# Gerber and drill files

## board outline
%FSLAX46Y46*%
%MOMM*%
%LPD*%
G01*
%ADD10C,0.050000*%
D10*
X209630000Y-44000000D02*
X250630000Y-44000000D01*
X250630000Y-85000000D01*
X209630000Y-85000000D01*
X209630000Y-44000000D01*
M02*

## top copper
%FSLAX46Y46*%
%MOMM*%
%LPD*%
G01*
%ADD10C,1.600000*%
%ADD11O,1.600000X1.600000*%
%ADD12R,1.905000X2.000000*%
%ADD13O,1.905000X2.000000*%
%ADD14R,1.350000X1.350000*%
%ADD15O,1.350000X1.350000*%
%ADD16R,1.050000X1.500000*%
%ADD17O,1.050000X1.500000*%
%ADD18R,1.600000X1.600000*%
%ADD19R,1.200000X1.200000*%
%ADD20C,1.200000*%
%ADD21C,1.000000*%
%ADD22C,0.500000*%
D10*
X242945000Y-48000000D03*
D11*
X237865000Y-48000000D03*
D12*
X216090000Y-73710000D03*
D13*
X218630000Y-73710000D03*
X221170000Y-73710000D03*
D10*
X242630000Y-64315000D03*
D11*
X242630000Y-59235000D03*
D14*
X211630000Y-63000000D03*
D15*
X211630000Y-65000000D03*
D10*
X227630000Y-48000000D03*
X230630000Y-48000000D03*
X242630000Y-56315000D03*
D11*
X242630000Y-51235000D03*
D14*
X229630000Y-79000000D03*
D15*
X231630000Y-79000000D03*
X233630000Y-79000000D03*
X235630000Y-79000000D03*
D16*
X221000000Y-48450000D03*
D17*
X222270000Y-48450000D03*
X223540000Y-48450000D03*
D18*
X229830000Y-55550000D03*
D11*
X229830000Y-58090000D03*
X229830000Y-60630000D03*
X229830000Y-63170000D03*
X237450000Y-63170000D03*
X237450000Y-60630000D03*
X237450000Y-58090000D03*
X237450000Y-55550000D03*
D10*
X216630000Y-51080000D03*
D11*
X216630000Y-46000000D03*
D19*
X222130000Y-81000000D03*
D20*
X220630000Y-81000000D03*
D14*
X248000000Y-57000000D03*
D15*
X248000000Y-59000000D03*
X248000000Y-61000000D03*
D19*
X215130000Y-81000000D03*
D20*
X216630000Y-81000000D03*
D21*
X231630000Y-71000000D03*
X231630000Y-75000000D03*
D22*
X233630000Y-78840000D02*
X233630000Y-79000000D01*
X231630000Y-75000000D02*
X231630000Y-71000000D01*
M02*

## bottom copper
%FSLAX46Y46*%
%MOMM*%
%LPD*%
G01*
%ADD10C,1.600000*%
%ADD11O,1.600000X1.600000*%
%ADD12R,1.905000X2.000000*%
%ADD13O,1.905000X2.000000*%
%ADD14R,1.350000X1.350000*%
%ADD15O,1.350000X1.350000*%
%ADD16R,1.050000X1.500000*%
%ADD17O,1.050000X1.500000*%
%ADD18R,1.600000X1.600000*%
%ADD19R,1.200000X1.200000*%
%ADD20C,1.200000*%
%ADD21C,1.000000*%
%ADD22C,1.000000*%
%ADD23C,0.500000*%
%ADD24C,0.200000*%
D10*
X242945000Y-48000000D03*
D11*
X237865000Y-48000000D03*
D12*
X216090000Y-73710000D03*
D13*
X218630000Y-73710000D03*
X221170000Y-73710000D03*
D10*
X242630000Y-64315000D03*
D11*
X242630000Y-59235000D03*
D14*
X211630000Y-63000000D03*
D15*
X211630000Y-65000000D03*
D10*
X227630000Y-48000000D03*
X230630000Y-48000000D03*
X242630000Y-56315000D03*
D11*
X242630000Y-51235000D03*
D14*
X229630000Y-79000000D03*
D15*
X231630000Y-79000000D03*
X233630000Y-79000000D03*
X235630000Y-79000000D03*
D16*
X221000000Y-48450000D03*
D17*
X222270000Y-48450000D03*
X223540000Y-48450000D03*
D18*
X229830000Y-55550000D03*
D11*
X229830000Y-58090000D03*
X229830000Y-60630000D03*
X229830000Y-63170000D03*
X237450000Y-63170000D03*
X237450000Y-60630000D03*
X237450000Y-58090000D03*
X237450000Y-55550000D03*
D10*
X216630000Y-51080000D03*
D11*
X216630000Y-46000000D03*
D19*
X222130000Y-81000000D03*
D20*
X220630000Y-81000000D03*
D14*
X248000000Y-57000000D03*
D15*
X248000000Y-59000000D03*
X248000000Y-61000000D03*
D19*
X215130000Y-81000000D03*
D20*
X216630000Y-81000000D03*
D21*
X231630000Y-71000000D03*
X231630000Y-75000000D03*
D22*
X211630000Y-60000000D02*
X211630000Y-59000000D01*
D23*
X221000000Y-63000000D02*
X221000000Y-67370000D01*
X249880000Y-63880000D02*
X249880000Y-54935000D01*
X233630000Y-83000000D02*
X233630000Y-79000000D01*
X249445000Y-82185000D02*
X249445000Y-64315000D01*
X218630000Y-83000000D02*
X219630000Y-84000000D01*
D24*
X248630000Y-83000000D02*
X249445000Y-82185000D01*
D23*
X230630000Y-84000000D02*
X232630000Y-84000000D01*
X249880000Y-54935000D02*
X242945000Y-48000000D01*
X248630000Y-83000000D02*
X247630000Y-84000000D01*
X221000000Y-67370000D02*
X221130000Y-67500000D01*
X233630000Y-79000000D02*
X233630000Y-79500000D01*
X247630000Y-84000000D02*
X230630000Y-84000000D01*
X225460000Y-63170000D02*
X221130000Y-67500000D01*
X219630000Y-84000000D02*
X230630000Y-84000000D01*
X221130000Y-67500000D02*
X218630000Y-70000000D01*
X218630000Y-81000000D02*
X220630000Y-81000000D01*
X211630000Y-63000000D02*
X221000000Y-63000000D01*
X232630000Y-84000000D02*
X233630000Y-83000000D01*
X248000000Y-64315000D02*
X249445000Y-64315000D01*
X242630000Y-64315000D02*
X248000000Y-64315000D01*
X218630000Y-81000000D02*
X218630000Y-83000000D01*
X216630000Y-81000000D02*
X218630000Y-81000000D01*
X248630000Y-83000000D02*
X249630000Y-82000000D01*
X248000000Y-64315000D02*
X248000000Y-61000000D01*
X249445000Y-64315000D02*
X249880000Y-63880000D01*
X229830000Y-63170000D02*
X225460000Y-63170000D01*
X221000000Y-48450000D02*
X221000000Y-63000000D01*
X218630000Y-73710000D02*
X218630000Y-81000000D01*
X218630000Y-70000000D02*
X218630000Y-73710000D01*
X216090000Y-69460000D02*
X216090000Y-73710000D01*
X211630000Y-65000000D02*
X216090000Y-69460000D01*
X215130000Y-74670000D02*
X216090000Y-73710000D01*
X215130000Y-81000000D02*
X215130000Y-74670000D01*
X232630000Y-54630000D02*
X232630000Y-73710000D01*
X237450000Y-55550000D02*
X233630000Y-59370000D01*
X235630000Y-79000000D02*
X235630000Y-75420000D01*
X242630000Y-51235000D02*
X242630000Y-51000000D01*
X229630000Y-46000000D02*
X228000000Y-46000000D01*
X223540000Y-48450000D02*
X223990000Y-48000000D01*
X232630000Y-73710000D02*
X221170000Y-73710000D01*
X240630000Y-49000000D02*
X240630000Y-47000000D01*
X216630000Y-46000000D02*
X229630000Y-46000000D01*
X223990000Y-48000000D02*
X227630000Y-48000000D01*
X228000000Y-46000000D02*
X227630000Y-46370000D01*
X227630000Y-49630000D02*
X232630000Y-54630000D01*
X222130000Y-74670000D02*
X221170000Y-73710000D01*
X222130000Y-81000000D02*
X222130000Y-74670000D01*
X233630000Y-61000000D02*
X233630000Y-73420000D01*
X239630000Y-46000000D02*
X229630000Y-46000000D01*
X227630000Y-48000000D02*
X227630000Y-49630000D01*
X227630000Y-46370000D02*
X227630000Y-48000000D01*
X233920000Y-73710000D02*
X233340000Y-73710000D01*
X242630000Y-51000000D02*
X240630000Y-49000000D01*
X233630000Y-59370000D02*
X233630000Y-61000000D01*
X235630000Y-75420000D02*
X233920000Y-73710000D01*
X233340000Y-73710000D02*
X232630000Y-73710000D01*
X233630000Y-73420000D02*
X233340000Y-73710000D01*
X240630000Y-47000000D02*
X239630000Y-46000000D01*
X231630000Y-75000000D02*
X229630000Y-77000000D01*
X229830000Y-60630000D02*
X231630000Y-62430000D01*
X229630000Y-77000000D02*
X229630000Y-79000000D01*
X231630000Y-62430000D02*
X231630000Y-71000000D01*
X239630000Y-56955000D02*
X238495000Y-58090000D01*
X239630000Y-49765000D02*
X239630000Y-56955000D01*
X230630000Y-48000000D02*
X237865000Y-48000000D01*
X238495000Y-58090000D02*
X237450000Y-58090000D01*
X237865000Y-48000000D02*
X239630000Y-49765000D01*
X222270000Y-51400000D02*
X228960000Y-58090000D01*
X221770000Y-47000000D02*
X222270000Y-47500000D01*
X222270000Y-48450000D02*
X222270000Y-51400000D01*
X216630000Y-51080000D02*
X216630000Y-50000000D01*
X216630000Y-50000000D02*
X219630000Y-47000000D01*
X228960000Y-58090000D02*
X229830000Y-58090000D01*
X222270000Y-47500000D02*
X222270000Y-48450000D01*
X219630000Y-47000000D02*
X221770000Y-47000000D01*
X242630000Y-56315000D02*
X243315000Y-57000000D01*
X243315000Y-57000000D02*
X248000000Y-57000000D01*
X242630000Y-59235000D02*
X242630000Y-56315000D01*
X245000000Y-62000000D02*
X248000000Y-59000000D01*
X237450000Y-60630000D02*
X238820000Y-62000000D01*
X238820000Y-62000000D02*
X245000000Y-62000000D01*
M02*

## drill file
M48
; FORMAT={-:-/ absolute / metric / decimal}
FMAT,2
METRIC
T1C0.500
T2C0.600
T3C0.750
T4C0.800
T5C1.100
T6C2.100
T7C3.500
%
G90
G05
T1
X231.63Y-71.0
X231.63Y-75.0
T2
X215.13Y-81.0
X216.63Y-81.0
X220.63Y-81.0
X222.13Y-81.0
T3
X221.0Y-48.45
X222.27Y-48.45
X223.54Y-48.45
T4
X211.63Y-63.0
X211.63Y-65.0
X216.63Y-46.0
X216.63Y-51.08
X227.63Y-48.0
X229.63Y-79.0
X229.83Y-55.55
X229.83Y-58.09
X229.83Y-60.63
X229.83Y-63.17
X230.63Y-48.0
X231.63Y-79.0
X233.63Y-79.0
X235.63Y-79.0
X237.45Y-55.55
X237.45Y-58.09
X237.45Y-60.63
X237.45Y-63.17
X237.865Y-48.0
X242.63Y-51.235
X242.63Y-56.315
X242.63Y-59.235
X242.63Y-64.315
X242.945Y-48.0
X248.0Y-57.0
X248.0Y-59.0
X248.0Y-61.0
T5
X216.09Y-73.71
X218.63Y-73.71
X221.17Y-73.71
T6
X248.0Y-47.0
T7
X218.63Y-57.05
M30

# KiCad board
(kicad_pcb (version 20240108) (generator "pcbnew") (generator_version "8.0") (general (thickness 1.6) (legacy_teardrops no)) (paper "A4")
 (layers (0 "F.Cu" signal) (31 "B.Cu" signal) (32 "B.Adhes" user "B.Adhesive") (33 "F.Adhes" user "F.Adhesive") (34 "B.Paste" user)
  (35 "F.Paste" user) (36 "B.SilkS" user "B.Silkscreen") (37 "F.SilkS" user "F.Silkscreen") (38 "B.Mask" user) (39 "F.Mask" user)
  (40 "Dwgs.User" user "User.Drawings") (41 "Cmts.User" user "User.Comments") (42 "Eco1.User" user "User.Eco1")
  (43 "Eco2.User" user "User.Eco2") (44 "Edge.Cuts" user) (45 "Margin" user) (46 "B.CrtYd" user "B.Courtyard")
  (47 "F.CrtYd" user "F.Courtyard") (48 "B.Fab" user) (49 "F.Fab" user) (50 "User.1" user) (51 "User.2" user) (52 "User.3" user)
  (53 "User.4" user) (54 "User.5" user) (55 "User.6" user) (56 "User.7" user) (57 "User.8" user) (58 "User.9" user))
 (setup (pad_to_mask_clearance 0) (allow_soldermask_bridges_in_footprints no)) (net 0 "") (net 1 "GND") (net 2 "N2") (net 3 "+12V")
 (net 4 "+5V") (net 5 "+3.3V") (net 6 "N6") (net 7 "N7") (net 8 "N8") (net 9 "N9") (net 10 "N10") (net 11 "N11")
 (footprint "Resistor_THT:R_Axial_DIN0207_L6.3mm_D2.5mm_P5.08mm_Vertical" (layer "F.Cu") (at 242.945 48 180)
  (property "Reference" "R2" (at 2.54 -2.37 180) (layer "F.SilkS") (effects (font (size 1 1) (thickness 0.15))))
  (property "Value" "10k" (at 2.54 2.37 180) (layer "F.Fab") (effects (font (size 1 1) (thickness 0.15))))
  (pad "1" thru_hole circle (at 0 0 180) (size 1.6 1.6) (drill 0.8) (layers "*.Cu" "*.Mask") (remove_unused_layers no) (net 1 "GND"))
  (pad "2" thru_hole oval (at 5.08 0 180) (size 1.6 1.6) (drill 0.8) (layers "*.Cu" "*.Mask") (remove_unused_layers no) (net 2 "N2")))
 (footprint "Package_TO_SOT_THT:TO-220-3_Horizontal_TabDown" (layer "F.Cu") (at 216.09 73.71)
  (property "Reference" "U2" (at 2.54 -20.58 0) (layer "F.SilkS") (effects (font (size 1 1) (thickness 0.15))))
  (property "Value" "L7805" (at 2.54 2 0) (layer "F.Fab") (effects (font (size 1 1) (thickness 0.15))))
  (pad "" np_thru_hole oval (at 2.54 -16.66) (size 3.5 3.5) (drill 3.5) (layers "*.Cu" "*.Mask"))
  (pad "1" thru_hole rect (at 0 0) (size 1.905 2) (drill 1.1) (layers "*.Cu" "*.Mask") (remove_unused_layers no) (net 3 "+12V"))
  (pad "2" thru_hole oval (at 2.54 0) (size 1.905 2) (drill 1.1) (layers "*.Cu" "*.Mask") (remove_unused_layers no) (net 1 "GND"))
  (pad "3" thru_hole oval (at 5.08 0) (size 1.905 2) (drill 1.1) (layers "*.Cu" "*.Mask") (remove_unused_layers no) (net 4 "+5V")))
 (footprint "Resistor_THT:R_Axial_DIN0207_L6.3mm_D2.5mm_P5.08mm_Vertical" (layer "F.Cu") (at 242.63 64.315 90)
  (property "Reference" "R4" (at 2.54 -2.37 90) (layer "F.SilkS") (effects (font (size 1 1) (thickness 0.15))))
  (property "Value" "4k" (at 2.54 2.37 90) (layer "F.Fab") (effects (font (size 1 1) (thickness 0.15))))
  (pad "1" thru_hole circle (at 0 0 90) (size 1.6 1.6) (drill 0.8) (layers "*.Cu" "*.Mask") (remove_unused_layers no) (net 1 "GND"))
  (pad "2" thru_hole oval (at 5.08 0 90) (size 1.6 1.6) (drill 0.8) (layers "*.Cu" "*.Mask") (remove_unused_layers no) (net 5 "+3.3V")))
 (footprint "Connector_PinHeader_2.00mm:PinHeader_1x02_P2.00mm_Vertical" (layer "F.Cu") (at 211.63 63)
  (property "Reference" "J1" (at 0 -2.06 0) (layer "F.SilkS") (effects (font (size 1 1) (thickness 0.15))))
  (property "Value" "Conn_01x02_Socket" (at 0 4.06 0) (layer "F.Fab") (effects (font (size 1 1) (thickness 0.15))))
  (pad "1" thru_hole rect (at 0 0) (size 1.35 1.35) (drill 0.8) (layers "*.Cu" "*.Mask") (remove_unused_layers no) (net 1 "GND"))
  (pad "2" thru_hole oval (at 0 2) (size 1.35 1.35) (drill 0.8) (layers "*.Cu" "*.Mask") (remove_unused_layers no) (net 3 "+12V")))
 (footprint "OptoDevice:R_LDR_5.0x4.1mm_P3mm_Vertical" (layer "F.Cu") (at 227.63 48)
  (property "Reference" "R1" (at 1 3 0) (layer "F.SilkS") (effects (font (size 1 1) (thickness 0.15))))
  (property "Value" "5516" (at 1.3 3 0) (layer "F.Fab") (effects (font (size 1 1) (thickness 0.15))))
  (pad "1" thru_hole circle (at 0 0) (size 1.6 1.6) (drill 0.8) (layers "*.Cu" "*.Mask") (remove_unused_layers no) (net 4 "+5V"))
  (pad "2" thru_hole circle (at 3 0) (size 1.6 1.6) (drill 0.8) (layers "*.Cu" "*.Mask") (remove_unused_layers no) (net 2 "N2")))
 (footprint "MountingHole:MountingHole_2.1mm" (layer "F.Cu") (at 248 47)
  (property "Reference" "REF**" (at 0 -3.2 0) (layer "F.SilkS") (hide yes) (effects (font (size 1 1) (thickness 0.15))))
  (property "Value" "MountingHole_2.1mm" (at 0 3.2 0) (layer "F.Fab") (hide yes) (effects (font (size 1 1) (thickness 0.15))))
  (pad "" np_thru_hole circle (at 0 0) (size 2.1 2.1) (drill 2.1) (layers "*.Cu" "*.Mask")))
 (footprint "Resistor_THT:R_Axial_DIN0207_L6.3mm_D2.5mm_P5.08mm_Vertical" (layer "F.Cu") (at 242.63 56.315 90)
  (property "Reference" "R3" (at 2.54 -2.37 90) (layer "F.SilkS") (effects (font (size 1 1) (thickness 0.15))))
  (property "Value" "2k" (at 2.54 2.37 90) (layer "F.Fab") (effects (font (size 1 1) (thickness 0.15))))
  (pad "1" thru_hole circle (at 0 0 90) (size 1.6 1.6) (drill 0.8) (layers "*.Cu" "*.Mask") (remove_unused_layers no) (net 5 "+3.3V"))
  (pad "2" thru_hole oval (at 5.08 0 90) (size 1.6 1.6) (drill 0.8) (layers "*.Cu" "*.Mask") (remove_unused_layers no) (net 4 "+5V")))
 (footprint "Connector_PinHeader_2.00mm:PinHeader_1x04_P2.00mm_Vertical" (layer "F.Cu") (at 229.63 79 90)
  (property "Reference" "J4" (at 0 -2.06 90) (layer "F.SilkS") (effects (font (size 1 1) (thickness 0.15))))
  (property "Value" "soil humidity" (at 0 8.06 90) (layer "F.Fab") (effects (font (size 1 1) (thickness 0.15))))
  (pad "1" thru_hole rect (at 0 0 90) (size 1.35 1.35) (drill 0.8) (layers "*.Cu" "*.Mask") (remove_unused_layers no) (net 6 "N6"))
  (pad "2" thru_hole oval (at 0 2 90) (size 1.35 1.35) (drill 0.8) (layers "*.Cu" "*.Mask") (remove_unused_layers no) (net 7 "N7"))
  (pad "3" thru_hole oval (at 0 4 90) (size 1.35 1.35) (drill 0.8) (layers "*.Cu" "*.Mask") (remove_unused_layers no) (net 1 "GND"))
  (pad "4" thru_hole oval (at 0 6 90) (size 1.35 1.35) (drill 0.8) (layers "*.Cu" "*.Mask") (remove_unused_layers no) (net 4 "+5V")))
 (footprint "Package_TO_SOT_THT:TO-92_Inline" (layer "F.Cu") (at 221 48.45)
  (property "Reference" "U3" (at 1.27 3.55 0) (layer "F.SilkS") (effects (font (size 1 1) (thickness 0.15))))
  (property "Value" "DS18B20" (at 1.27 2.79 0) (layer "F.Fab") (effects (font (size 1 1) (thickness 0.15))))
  (pad "1" thru_hole rect (at 0 0) (size 1.05 1.5) (drill 0.75) (layers "*.Cu" "*.Mask") (remove_unused_layers no) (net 1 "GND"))
  (pad "2" thru_hole oval (at 1.27 0) (size 1.05 1.5) (drill 0.75) (layers "*.Cu" "*.Mask") (remove_unused_layers no) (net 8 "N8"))
  (pad "3" thru_hole oval (at 2.54 0) (size 1.05 1.5) (drill 0.75) (layers "*.Cu" "*.Mask") (remove_unused_layers no) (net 4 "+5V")))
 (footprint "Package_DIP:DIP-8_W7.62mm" (layer "F.Cu") (at 229.83 55.55)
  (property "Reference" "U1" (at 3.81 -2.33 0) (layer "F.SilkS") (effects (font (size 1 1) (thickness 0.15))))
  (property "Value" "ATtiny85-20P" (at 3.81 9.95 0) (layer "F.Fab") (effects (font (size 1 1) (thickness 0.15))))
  (pad "1" thru_hole rect (at 0 0) (size 1.6 1.6) (drill 0.8) (layers "*.Cu" "*.Mask") (remove_unused_layers no) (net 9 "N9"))
  (pad "2" thru_hole oval (at 0 2.54) (size 1.6 1.6) (drill 0.8) (layers "*.Cu" "*.Mask") (remove_unused_layers no) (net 8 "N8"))
  (pad "3" thru_hole oval (at 0 5.08) (size 1.6 1.6) (drill 0.8) (layers "*.Cu" "*.Mask") (remove_unused_layers no) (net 6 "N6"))
  (pad "4" thru_hole oval (at 0 7.62) (size 1.6 1.6) (drill 0.8) (layers "*.Cu" "*.Mask") (remove_unused_layers no) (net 1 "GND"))
  (pad "5" thru_hole oval (at 7.62 7.62) (size 1.6 1.6) (drill 0.8) (layers "*.Cu" "*.Mask") (remove_unused_layers no) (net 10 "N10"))
  (pad "6" thru_hole oval (at 7.62 5.08) (size 1.6 1.6) (drill 0.8) (layers "*.Cu" "*.Mask") (remove_unused_layers no) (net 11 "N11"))
  (pad "7" thru_hole oval (at 7.62 2.54) (size 1.6 1.6) (drill 0.8) (layers "*.Cu" "*.Mask") (remove_unused_layers no) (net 2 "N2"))
  (pad "8" thru_hole oval (at 7.62 0) (size 1.6 1.6) (drill 0.8) (layers "*.Cu" "*.Mask") (remove_unused_layers no) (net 4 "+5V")))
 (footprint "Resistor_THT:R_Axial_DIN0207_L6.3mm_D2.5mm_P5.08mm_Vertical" (layer "F.Cu") (at 216.63 51.08 90)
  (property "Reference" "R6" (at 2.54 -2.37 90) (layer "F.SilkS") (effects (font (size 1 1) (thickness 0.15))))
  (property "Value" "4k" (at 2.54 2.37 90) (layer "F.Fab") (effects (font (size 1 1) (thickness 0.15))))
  (pad "1" thru_hole circle (at 0 0 90) (size 1.6 1.6) (drill 0.8) (layers "*.Cu" "*.Mask") (remove_unused_layers no) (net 8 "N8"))
  (pad "2" thru_hole oval (at 5.08 0 90) (size 1.6 1.6) (drill 0.8) (layers "*.Cu" "*.Mask") (remove_unused_layers no) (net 4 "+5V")))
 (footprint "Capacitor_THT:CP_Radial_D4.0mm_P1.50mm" (layer "F.Cu") (at 222.13 81 180)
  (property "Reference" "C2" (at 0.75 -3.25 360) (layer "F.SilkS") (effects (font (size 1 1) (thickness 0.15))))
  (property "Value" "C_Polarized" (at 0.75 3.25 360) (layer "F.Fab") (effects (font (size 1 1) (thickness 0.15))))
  (pad "1" thru_hole rect (at 0 0 180) (size 1.2 1.2) (drill 0.6) (layers "*.Cu" "*.Mask") (remove_unused_layers no) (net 4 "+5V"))
  (pad "2" thru_hole circle (at 1.5 0 180) (size 1.2 1.2) (drill 0.6) (layers "*.Cu" "*.Mask") (remove_unused_layers no) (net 1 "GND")))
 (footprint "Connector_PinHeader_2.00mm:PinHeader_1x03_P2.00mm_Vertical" (layer "F.Cu") (at 248 57)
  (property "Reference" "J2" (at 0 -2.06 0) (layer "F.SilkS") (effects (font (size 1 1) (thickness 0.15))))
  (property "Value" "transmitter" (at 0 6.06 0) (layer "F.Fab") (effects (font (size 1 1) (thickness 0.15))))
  (pad "1" thru_hole rect (at 0 0) (size 1.35 1.35) (drill 0.8) (layers "*.Cu" "*.Mask") (remove_unused_layers no) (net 5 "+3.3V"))
  (pad "2" thru_hole oval (at 0 2) (size 1.35 1.35) (drill 0.8) (layers "*.Cu" "*.Mask") (remove_unused_layers no) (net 11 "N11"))
  (pad "3" thru_hole oval (at 0 4) (size 1.35 1.35) (drill 0.8) (layers "*.Cu" "*.Mask") (remove_unused_layers no) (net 1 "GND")))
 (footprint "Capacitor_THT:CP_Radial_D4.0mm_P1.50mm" (layer "F.Cu") (at 215.13 81)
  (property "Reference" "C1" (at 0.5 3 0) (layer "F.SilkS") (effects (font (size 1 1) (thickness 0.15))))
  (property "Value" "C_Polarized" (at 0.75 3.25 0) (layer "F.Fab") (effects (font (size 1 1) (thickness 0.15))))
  (pad "1" thru_hole rect (at 0 0) (size 1.2 1.2) (drill 0.6) (layers "*.Cu" "*.Mask") (remove_unused_layers no) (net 3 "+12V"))
  (pad "2" thru_hole circle (at 1.5 0) (size 1.2 1.2) (drill 0.6) (layers "*.Cu" "*.Mask") (remove_unused_layers no) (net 1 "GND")))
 (gr_rect (start 209.63 44) (end 250.63 85) (stroke (width 0.05) (type default)) (fill none) (layer "Edge.Cuts"))
 (segment (start 211.63 60) (end 211.63 59) (width 1) (layer "B.Cu") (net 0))
 (segment (start 233.63 78.84) (end 233.63 79) (width 0.5) (layer "F.Cu") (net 1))
 (segment (start 221 63) (end 221 67.37) (width 0.5) (layer "B.Cu") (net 1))
 (segment (start 249.88 63.88) (end 249.88 54.935) (width 0.5) (layer "B.Cu") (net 1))
 (segment (start 233.63 83) (end 233.63 79) (width 0.5) (layer "B.Cu") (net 1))
 (segment (start 249.445 82.185) (end 249.445 64.315) (width 0.5) (layer "B.Cu") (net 1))
 (segment (start 218.63 83) (end 219.63 84) (width 0.5) (layer "B.Cu") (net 1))
 (segment (start 248.63 83) (end 249.445 82.185) (width 0.2) (layer "B.Cu") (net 1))
 (segment (start 230.63 84) (end 232.63 84) (width 0.5) (layer "B.Cu") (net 1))
 (segment (start 249.88 54.935) (end 242.945 48) (width 0.5) (layer "B.Cu") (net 1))
 (segment (start 248.63 83) (end 247.63 84) (width 0.5) (layer "B.Cu") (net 1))
 (segment (start 221 67.37) (end 221.13 67.5) (width 0.5) (layer "B.Cu") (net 1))
 (segment (start 233.63 79) (end 233.63 79.5) (width 0.5) (layer "B.Cu") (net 1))
 (segment (start 247.63 84) (end 230.63 84) (width 0.5) (layer "B.Cu") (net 1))
 (segment (start 225.46 63.17) (end 221.13 67.5) (width 0.5) (layer "B.Cu") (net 1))
 (segment (start 219.63 84) (end 230.63 84) (width 0.5) (layer "B.Cu") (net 1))
 (segment (start 221.13 67.5) (end 218.63 70) (width 0.5) (layer "B.Cu") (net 1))
 (segment (start 218.63 81) (end 220.63 81) (width 0.5) (layer "B.Cu") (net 1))
 (segment (start 211.63 63) (end 221 63) (width 0.5) (layer "B.Cu") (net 1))
 (segment (start 232.63 84) (end 233.63 83) (width 0.5) (layer "B.Cu") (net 1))
 (segment (start 248 64.315) (end 249.445 64.315) (width 0.5) (layer "B.Cu") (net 1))
 (segment (start 242.63 64.315) (end 248 64.315) (width 0.5) (layer "B.Cu") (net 1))
 (segment (start 218.63 81) (end 218.63 83) (width 0.5) (layer "B.Cu") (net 1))
 (segment (start 216.63 81) (end 218.63 81) (width 0.5) (layer "B.Cu") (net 1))
 (segment (start 248.63 83) (end 249.63 82) (width 0.5) (layer "B.Cu") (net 1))
 (segment (start 248 64.315) (end 248 61) (width 0.5) (layer "B.Cu") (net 1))
 (segment (start 249.445 64.315) (end 249.88 63.88) (width 0.5) (layer "B.Cu") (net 1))
 (segment (start 229.83 63.17) (end 225.46 63.17) (width 0.5) (layer "B.Cu") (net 1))
 (segment (start 221 48.45) (end 221 63) (width 0.5) (layer "B.Cu") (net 1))
 (segment (start 218.63 73.71) (end 218.63 81) (width 0.5) (layer "B.Cu") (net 1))
 (segment (start 218.63 70) (end 218.63 73.71) (width 0.5) (layer "B.Cu") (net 1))
 (segment (start 216.09 69.46) (end 216.09 73.71) (width 0.5) (layer "B.Cu") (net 3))
 (segment (start 211.63 65) (end 216.09 69.46) (width 0.5) (layer "B.Cu") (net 3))
 (segment (start 215.13 74.67) (end 216.09 73.71) (width 0.5) (layer "B.Cu") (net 3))
 (segment (start 215.13 81) (end 215.13 74.67) (width 0.5) (layer "B.Cu") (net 3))
 (segment (start 232.63 54.63) (end 232.63 73.71) (width 0.5) (layer "B.Cu") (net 4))
 (segment (start 237.45 55.55) (end 233.63 59.37) (width 0.5) (layer "B.Cu") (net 4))
 (segment (start 235.63 79) (end 235.63 75.42) (width 0.5) (layer "B.Cu") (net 4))
 (segment (start 242.63 51.235) (end 242.63 51) (width 0.5) (layer "B.Cu") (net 4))
 (segment (start 229.63 46) (end 228 46) (width 0.5) (layer "B.Cu") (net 4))
 (segment (start 223.54 48.45) (end 223.99 48) (width 0.5) (layer "B.Cu") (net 4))
 (segment (start 232.63 73.71) (end 221.17 73.71) (width 0.5) (layer "B.Cu") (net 4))
 (segment (start 240.63 49) (end 240.63 47) (width 0.5) (layer "B.Cu") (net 4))
 (segment (start 216.63 46) (end 229.63 46) (width 0.5) (layer "B.Cu") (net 4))
 (segment (start 223.99 48) (end 227.63 48) (width 0.5) (layer "B.Cu") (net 4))
 (segment (start 228 46) (end 227.63 46.37) (width 0.5) (layer "B.Cu") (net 4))
 (segment (start 227.63 49.63) (end 232.63 54.63) (width 0.5) (layer "B.Cu") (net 4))
 (segment (start 222.13 74.67) (end 221.17 73.71) (width 0.5) (layer "B.Cu") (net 4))
 (segment (start 222.13 81) (end 222.13 74.67) (width 0.5) (layer "B.Cu") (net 4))
 (segment (start 233.63 61) (end 233.63 73.42) (width 0.5) (layer "B.Cu") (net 4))
 (segment (start 239.63 46) (end 229.63 46) (width 0.5) (layer "B.Cu") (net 4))
 (segment (start 227.63 48) (end 227.63 49.63) (width 0.5) (layer "B.Cu") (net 4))
 (segment (start 227.63 46.37) (end 227.63 48) (width 0.5) (layer "B.Cu") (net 4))
 (segment (start 233.92 73.71) (end 233.34 73.71) (width 0.5) (layer "B.Cu") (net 4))
 (segment (start 242.63 51) (end 240.63 49) (width 0.5) (layer "B.Cu") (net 4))
 (segment (start 233.63 59.37) (end 233.63 61) (width 0.5) (layer "B.Cu") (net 4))
 (segment (start 235.63 75.42) (end 233.92 73.71) (width 0.5) (layer "B.Cu") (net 4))
 (segment (start 233.34 73.71) (end 232.63 73.71) (width 0.5) (layer "B.Cu") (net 4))
 (segment (start 233.63 73.42) (end 233.34 73.71) (width 0.5) (layer "B.Cu") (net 4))
 (segment (start 240.63 47) (end 239.63 46) (width 0.5) (layer "B.Cu") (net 4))
 (segment (start 231.63 75) (end 231.63 71) (width 0.5) (layer "F.Cu") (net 6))
 (via (at 231.63 71) (size 1) (drill 0.5) (layers "F.Cu" "B.Cu") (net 6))
 (via (at 231.63 75) (size 1) (drill 0.5) (layers "F.Cu" "B.Cu") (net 6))
 (segment (start 231.63 75) (end 229.63 77) (width 0.5) (layer "B.Cu") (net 6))
 (segment (start 229.83 60.63) (end 231.63 62.43) (width 0.5) (layer "B.Cu") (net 6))
 (segment (start 229.63 77) (end 229.63 79) (width 0.5) (layer "B.Cu") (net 6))
 (segment (start 231.63 62.43) (end 231.63 71) (width 0.5) (layer "B.Cu") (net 6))
 (segment (start 239.63 56.955) (end 238.495 58.09) (width 0.5) (layer "B.Cu") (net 2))
 (segment (start 239.63 49.765) (end 239.63 56.955) (width 0.5) (layer "B.Cu") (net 2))
 (segment (start 230.63 48) (end 237.865 48) (width 0.5) (layer "B.Cu") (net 2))
 (segment (start 238.495 58.09) (end 237.45 58.09) (width 0.5) (layer "B.Cu") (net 2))
 (segment (start 237.865 48) (end 239.63 49.765) (width 0.5) (layer "B.Cu") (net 2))
 (segment (start 222.27 51.4) (end 228.96 58.09) (width 0.5) (layer "B.Cu") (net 8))
 (segment (start 221.77 47) (end 222.27 47.5) (width 0.5) (layer "B.Cu") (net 8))
 (segment (start 222.27 48.45) (end 222.27 51.4) (width 0.5) (layer "B.Cu") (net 8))
 (segment (start 216.63 51.08) (end 216.63 50) (width 0.5) (layer "B.Cu") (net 8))
 (segment (start 216.63 50) (end 219.63 47) (width 0.5) (layer "B.Cu") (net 8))
 (segment (start 228.96 58.09) (end 229.83 58.09) (width 0.5) (layer "B.Cu") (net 8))
 (segment (start 222.27 47.5) (end 222.27 48.45) (width 0.5) (layer "B.Cu") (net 8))
 (segment (start 219.63 47) (end 221.77 47) (width 0.5) (layer "B.Cu") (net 8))
 (segment (start 242.63 56.315) (end 243.315 57) (width 0.5) (layer "B.Cu") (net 5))
 (segment (start 243.315 57) (end 248 57) (width 0.5) (layer "B.Cu") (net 5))
 (segment (start 242.63 59.235) (end 242.63 56.315) (width 0.5) (layer "B.Cu") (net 5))
 (segment (start 245 62) (end 248 59) (width 0.5) (layer "B.Cu") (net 11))
 (segment (start 237.45 60.63) (end 238.82 62) (width 0.5) (layer "B.Cu") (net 11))
 (segment (start 238.82 62) (end 245 62) (width 0.5) (layer "B.Cu") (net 11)))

